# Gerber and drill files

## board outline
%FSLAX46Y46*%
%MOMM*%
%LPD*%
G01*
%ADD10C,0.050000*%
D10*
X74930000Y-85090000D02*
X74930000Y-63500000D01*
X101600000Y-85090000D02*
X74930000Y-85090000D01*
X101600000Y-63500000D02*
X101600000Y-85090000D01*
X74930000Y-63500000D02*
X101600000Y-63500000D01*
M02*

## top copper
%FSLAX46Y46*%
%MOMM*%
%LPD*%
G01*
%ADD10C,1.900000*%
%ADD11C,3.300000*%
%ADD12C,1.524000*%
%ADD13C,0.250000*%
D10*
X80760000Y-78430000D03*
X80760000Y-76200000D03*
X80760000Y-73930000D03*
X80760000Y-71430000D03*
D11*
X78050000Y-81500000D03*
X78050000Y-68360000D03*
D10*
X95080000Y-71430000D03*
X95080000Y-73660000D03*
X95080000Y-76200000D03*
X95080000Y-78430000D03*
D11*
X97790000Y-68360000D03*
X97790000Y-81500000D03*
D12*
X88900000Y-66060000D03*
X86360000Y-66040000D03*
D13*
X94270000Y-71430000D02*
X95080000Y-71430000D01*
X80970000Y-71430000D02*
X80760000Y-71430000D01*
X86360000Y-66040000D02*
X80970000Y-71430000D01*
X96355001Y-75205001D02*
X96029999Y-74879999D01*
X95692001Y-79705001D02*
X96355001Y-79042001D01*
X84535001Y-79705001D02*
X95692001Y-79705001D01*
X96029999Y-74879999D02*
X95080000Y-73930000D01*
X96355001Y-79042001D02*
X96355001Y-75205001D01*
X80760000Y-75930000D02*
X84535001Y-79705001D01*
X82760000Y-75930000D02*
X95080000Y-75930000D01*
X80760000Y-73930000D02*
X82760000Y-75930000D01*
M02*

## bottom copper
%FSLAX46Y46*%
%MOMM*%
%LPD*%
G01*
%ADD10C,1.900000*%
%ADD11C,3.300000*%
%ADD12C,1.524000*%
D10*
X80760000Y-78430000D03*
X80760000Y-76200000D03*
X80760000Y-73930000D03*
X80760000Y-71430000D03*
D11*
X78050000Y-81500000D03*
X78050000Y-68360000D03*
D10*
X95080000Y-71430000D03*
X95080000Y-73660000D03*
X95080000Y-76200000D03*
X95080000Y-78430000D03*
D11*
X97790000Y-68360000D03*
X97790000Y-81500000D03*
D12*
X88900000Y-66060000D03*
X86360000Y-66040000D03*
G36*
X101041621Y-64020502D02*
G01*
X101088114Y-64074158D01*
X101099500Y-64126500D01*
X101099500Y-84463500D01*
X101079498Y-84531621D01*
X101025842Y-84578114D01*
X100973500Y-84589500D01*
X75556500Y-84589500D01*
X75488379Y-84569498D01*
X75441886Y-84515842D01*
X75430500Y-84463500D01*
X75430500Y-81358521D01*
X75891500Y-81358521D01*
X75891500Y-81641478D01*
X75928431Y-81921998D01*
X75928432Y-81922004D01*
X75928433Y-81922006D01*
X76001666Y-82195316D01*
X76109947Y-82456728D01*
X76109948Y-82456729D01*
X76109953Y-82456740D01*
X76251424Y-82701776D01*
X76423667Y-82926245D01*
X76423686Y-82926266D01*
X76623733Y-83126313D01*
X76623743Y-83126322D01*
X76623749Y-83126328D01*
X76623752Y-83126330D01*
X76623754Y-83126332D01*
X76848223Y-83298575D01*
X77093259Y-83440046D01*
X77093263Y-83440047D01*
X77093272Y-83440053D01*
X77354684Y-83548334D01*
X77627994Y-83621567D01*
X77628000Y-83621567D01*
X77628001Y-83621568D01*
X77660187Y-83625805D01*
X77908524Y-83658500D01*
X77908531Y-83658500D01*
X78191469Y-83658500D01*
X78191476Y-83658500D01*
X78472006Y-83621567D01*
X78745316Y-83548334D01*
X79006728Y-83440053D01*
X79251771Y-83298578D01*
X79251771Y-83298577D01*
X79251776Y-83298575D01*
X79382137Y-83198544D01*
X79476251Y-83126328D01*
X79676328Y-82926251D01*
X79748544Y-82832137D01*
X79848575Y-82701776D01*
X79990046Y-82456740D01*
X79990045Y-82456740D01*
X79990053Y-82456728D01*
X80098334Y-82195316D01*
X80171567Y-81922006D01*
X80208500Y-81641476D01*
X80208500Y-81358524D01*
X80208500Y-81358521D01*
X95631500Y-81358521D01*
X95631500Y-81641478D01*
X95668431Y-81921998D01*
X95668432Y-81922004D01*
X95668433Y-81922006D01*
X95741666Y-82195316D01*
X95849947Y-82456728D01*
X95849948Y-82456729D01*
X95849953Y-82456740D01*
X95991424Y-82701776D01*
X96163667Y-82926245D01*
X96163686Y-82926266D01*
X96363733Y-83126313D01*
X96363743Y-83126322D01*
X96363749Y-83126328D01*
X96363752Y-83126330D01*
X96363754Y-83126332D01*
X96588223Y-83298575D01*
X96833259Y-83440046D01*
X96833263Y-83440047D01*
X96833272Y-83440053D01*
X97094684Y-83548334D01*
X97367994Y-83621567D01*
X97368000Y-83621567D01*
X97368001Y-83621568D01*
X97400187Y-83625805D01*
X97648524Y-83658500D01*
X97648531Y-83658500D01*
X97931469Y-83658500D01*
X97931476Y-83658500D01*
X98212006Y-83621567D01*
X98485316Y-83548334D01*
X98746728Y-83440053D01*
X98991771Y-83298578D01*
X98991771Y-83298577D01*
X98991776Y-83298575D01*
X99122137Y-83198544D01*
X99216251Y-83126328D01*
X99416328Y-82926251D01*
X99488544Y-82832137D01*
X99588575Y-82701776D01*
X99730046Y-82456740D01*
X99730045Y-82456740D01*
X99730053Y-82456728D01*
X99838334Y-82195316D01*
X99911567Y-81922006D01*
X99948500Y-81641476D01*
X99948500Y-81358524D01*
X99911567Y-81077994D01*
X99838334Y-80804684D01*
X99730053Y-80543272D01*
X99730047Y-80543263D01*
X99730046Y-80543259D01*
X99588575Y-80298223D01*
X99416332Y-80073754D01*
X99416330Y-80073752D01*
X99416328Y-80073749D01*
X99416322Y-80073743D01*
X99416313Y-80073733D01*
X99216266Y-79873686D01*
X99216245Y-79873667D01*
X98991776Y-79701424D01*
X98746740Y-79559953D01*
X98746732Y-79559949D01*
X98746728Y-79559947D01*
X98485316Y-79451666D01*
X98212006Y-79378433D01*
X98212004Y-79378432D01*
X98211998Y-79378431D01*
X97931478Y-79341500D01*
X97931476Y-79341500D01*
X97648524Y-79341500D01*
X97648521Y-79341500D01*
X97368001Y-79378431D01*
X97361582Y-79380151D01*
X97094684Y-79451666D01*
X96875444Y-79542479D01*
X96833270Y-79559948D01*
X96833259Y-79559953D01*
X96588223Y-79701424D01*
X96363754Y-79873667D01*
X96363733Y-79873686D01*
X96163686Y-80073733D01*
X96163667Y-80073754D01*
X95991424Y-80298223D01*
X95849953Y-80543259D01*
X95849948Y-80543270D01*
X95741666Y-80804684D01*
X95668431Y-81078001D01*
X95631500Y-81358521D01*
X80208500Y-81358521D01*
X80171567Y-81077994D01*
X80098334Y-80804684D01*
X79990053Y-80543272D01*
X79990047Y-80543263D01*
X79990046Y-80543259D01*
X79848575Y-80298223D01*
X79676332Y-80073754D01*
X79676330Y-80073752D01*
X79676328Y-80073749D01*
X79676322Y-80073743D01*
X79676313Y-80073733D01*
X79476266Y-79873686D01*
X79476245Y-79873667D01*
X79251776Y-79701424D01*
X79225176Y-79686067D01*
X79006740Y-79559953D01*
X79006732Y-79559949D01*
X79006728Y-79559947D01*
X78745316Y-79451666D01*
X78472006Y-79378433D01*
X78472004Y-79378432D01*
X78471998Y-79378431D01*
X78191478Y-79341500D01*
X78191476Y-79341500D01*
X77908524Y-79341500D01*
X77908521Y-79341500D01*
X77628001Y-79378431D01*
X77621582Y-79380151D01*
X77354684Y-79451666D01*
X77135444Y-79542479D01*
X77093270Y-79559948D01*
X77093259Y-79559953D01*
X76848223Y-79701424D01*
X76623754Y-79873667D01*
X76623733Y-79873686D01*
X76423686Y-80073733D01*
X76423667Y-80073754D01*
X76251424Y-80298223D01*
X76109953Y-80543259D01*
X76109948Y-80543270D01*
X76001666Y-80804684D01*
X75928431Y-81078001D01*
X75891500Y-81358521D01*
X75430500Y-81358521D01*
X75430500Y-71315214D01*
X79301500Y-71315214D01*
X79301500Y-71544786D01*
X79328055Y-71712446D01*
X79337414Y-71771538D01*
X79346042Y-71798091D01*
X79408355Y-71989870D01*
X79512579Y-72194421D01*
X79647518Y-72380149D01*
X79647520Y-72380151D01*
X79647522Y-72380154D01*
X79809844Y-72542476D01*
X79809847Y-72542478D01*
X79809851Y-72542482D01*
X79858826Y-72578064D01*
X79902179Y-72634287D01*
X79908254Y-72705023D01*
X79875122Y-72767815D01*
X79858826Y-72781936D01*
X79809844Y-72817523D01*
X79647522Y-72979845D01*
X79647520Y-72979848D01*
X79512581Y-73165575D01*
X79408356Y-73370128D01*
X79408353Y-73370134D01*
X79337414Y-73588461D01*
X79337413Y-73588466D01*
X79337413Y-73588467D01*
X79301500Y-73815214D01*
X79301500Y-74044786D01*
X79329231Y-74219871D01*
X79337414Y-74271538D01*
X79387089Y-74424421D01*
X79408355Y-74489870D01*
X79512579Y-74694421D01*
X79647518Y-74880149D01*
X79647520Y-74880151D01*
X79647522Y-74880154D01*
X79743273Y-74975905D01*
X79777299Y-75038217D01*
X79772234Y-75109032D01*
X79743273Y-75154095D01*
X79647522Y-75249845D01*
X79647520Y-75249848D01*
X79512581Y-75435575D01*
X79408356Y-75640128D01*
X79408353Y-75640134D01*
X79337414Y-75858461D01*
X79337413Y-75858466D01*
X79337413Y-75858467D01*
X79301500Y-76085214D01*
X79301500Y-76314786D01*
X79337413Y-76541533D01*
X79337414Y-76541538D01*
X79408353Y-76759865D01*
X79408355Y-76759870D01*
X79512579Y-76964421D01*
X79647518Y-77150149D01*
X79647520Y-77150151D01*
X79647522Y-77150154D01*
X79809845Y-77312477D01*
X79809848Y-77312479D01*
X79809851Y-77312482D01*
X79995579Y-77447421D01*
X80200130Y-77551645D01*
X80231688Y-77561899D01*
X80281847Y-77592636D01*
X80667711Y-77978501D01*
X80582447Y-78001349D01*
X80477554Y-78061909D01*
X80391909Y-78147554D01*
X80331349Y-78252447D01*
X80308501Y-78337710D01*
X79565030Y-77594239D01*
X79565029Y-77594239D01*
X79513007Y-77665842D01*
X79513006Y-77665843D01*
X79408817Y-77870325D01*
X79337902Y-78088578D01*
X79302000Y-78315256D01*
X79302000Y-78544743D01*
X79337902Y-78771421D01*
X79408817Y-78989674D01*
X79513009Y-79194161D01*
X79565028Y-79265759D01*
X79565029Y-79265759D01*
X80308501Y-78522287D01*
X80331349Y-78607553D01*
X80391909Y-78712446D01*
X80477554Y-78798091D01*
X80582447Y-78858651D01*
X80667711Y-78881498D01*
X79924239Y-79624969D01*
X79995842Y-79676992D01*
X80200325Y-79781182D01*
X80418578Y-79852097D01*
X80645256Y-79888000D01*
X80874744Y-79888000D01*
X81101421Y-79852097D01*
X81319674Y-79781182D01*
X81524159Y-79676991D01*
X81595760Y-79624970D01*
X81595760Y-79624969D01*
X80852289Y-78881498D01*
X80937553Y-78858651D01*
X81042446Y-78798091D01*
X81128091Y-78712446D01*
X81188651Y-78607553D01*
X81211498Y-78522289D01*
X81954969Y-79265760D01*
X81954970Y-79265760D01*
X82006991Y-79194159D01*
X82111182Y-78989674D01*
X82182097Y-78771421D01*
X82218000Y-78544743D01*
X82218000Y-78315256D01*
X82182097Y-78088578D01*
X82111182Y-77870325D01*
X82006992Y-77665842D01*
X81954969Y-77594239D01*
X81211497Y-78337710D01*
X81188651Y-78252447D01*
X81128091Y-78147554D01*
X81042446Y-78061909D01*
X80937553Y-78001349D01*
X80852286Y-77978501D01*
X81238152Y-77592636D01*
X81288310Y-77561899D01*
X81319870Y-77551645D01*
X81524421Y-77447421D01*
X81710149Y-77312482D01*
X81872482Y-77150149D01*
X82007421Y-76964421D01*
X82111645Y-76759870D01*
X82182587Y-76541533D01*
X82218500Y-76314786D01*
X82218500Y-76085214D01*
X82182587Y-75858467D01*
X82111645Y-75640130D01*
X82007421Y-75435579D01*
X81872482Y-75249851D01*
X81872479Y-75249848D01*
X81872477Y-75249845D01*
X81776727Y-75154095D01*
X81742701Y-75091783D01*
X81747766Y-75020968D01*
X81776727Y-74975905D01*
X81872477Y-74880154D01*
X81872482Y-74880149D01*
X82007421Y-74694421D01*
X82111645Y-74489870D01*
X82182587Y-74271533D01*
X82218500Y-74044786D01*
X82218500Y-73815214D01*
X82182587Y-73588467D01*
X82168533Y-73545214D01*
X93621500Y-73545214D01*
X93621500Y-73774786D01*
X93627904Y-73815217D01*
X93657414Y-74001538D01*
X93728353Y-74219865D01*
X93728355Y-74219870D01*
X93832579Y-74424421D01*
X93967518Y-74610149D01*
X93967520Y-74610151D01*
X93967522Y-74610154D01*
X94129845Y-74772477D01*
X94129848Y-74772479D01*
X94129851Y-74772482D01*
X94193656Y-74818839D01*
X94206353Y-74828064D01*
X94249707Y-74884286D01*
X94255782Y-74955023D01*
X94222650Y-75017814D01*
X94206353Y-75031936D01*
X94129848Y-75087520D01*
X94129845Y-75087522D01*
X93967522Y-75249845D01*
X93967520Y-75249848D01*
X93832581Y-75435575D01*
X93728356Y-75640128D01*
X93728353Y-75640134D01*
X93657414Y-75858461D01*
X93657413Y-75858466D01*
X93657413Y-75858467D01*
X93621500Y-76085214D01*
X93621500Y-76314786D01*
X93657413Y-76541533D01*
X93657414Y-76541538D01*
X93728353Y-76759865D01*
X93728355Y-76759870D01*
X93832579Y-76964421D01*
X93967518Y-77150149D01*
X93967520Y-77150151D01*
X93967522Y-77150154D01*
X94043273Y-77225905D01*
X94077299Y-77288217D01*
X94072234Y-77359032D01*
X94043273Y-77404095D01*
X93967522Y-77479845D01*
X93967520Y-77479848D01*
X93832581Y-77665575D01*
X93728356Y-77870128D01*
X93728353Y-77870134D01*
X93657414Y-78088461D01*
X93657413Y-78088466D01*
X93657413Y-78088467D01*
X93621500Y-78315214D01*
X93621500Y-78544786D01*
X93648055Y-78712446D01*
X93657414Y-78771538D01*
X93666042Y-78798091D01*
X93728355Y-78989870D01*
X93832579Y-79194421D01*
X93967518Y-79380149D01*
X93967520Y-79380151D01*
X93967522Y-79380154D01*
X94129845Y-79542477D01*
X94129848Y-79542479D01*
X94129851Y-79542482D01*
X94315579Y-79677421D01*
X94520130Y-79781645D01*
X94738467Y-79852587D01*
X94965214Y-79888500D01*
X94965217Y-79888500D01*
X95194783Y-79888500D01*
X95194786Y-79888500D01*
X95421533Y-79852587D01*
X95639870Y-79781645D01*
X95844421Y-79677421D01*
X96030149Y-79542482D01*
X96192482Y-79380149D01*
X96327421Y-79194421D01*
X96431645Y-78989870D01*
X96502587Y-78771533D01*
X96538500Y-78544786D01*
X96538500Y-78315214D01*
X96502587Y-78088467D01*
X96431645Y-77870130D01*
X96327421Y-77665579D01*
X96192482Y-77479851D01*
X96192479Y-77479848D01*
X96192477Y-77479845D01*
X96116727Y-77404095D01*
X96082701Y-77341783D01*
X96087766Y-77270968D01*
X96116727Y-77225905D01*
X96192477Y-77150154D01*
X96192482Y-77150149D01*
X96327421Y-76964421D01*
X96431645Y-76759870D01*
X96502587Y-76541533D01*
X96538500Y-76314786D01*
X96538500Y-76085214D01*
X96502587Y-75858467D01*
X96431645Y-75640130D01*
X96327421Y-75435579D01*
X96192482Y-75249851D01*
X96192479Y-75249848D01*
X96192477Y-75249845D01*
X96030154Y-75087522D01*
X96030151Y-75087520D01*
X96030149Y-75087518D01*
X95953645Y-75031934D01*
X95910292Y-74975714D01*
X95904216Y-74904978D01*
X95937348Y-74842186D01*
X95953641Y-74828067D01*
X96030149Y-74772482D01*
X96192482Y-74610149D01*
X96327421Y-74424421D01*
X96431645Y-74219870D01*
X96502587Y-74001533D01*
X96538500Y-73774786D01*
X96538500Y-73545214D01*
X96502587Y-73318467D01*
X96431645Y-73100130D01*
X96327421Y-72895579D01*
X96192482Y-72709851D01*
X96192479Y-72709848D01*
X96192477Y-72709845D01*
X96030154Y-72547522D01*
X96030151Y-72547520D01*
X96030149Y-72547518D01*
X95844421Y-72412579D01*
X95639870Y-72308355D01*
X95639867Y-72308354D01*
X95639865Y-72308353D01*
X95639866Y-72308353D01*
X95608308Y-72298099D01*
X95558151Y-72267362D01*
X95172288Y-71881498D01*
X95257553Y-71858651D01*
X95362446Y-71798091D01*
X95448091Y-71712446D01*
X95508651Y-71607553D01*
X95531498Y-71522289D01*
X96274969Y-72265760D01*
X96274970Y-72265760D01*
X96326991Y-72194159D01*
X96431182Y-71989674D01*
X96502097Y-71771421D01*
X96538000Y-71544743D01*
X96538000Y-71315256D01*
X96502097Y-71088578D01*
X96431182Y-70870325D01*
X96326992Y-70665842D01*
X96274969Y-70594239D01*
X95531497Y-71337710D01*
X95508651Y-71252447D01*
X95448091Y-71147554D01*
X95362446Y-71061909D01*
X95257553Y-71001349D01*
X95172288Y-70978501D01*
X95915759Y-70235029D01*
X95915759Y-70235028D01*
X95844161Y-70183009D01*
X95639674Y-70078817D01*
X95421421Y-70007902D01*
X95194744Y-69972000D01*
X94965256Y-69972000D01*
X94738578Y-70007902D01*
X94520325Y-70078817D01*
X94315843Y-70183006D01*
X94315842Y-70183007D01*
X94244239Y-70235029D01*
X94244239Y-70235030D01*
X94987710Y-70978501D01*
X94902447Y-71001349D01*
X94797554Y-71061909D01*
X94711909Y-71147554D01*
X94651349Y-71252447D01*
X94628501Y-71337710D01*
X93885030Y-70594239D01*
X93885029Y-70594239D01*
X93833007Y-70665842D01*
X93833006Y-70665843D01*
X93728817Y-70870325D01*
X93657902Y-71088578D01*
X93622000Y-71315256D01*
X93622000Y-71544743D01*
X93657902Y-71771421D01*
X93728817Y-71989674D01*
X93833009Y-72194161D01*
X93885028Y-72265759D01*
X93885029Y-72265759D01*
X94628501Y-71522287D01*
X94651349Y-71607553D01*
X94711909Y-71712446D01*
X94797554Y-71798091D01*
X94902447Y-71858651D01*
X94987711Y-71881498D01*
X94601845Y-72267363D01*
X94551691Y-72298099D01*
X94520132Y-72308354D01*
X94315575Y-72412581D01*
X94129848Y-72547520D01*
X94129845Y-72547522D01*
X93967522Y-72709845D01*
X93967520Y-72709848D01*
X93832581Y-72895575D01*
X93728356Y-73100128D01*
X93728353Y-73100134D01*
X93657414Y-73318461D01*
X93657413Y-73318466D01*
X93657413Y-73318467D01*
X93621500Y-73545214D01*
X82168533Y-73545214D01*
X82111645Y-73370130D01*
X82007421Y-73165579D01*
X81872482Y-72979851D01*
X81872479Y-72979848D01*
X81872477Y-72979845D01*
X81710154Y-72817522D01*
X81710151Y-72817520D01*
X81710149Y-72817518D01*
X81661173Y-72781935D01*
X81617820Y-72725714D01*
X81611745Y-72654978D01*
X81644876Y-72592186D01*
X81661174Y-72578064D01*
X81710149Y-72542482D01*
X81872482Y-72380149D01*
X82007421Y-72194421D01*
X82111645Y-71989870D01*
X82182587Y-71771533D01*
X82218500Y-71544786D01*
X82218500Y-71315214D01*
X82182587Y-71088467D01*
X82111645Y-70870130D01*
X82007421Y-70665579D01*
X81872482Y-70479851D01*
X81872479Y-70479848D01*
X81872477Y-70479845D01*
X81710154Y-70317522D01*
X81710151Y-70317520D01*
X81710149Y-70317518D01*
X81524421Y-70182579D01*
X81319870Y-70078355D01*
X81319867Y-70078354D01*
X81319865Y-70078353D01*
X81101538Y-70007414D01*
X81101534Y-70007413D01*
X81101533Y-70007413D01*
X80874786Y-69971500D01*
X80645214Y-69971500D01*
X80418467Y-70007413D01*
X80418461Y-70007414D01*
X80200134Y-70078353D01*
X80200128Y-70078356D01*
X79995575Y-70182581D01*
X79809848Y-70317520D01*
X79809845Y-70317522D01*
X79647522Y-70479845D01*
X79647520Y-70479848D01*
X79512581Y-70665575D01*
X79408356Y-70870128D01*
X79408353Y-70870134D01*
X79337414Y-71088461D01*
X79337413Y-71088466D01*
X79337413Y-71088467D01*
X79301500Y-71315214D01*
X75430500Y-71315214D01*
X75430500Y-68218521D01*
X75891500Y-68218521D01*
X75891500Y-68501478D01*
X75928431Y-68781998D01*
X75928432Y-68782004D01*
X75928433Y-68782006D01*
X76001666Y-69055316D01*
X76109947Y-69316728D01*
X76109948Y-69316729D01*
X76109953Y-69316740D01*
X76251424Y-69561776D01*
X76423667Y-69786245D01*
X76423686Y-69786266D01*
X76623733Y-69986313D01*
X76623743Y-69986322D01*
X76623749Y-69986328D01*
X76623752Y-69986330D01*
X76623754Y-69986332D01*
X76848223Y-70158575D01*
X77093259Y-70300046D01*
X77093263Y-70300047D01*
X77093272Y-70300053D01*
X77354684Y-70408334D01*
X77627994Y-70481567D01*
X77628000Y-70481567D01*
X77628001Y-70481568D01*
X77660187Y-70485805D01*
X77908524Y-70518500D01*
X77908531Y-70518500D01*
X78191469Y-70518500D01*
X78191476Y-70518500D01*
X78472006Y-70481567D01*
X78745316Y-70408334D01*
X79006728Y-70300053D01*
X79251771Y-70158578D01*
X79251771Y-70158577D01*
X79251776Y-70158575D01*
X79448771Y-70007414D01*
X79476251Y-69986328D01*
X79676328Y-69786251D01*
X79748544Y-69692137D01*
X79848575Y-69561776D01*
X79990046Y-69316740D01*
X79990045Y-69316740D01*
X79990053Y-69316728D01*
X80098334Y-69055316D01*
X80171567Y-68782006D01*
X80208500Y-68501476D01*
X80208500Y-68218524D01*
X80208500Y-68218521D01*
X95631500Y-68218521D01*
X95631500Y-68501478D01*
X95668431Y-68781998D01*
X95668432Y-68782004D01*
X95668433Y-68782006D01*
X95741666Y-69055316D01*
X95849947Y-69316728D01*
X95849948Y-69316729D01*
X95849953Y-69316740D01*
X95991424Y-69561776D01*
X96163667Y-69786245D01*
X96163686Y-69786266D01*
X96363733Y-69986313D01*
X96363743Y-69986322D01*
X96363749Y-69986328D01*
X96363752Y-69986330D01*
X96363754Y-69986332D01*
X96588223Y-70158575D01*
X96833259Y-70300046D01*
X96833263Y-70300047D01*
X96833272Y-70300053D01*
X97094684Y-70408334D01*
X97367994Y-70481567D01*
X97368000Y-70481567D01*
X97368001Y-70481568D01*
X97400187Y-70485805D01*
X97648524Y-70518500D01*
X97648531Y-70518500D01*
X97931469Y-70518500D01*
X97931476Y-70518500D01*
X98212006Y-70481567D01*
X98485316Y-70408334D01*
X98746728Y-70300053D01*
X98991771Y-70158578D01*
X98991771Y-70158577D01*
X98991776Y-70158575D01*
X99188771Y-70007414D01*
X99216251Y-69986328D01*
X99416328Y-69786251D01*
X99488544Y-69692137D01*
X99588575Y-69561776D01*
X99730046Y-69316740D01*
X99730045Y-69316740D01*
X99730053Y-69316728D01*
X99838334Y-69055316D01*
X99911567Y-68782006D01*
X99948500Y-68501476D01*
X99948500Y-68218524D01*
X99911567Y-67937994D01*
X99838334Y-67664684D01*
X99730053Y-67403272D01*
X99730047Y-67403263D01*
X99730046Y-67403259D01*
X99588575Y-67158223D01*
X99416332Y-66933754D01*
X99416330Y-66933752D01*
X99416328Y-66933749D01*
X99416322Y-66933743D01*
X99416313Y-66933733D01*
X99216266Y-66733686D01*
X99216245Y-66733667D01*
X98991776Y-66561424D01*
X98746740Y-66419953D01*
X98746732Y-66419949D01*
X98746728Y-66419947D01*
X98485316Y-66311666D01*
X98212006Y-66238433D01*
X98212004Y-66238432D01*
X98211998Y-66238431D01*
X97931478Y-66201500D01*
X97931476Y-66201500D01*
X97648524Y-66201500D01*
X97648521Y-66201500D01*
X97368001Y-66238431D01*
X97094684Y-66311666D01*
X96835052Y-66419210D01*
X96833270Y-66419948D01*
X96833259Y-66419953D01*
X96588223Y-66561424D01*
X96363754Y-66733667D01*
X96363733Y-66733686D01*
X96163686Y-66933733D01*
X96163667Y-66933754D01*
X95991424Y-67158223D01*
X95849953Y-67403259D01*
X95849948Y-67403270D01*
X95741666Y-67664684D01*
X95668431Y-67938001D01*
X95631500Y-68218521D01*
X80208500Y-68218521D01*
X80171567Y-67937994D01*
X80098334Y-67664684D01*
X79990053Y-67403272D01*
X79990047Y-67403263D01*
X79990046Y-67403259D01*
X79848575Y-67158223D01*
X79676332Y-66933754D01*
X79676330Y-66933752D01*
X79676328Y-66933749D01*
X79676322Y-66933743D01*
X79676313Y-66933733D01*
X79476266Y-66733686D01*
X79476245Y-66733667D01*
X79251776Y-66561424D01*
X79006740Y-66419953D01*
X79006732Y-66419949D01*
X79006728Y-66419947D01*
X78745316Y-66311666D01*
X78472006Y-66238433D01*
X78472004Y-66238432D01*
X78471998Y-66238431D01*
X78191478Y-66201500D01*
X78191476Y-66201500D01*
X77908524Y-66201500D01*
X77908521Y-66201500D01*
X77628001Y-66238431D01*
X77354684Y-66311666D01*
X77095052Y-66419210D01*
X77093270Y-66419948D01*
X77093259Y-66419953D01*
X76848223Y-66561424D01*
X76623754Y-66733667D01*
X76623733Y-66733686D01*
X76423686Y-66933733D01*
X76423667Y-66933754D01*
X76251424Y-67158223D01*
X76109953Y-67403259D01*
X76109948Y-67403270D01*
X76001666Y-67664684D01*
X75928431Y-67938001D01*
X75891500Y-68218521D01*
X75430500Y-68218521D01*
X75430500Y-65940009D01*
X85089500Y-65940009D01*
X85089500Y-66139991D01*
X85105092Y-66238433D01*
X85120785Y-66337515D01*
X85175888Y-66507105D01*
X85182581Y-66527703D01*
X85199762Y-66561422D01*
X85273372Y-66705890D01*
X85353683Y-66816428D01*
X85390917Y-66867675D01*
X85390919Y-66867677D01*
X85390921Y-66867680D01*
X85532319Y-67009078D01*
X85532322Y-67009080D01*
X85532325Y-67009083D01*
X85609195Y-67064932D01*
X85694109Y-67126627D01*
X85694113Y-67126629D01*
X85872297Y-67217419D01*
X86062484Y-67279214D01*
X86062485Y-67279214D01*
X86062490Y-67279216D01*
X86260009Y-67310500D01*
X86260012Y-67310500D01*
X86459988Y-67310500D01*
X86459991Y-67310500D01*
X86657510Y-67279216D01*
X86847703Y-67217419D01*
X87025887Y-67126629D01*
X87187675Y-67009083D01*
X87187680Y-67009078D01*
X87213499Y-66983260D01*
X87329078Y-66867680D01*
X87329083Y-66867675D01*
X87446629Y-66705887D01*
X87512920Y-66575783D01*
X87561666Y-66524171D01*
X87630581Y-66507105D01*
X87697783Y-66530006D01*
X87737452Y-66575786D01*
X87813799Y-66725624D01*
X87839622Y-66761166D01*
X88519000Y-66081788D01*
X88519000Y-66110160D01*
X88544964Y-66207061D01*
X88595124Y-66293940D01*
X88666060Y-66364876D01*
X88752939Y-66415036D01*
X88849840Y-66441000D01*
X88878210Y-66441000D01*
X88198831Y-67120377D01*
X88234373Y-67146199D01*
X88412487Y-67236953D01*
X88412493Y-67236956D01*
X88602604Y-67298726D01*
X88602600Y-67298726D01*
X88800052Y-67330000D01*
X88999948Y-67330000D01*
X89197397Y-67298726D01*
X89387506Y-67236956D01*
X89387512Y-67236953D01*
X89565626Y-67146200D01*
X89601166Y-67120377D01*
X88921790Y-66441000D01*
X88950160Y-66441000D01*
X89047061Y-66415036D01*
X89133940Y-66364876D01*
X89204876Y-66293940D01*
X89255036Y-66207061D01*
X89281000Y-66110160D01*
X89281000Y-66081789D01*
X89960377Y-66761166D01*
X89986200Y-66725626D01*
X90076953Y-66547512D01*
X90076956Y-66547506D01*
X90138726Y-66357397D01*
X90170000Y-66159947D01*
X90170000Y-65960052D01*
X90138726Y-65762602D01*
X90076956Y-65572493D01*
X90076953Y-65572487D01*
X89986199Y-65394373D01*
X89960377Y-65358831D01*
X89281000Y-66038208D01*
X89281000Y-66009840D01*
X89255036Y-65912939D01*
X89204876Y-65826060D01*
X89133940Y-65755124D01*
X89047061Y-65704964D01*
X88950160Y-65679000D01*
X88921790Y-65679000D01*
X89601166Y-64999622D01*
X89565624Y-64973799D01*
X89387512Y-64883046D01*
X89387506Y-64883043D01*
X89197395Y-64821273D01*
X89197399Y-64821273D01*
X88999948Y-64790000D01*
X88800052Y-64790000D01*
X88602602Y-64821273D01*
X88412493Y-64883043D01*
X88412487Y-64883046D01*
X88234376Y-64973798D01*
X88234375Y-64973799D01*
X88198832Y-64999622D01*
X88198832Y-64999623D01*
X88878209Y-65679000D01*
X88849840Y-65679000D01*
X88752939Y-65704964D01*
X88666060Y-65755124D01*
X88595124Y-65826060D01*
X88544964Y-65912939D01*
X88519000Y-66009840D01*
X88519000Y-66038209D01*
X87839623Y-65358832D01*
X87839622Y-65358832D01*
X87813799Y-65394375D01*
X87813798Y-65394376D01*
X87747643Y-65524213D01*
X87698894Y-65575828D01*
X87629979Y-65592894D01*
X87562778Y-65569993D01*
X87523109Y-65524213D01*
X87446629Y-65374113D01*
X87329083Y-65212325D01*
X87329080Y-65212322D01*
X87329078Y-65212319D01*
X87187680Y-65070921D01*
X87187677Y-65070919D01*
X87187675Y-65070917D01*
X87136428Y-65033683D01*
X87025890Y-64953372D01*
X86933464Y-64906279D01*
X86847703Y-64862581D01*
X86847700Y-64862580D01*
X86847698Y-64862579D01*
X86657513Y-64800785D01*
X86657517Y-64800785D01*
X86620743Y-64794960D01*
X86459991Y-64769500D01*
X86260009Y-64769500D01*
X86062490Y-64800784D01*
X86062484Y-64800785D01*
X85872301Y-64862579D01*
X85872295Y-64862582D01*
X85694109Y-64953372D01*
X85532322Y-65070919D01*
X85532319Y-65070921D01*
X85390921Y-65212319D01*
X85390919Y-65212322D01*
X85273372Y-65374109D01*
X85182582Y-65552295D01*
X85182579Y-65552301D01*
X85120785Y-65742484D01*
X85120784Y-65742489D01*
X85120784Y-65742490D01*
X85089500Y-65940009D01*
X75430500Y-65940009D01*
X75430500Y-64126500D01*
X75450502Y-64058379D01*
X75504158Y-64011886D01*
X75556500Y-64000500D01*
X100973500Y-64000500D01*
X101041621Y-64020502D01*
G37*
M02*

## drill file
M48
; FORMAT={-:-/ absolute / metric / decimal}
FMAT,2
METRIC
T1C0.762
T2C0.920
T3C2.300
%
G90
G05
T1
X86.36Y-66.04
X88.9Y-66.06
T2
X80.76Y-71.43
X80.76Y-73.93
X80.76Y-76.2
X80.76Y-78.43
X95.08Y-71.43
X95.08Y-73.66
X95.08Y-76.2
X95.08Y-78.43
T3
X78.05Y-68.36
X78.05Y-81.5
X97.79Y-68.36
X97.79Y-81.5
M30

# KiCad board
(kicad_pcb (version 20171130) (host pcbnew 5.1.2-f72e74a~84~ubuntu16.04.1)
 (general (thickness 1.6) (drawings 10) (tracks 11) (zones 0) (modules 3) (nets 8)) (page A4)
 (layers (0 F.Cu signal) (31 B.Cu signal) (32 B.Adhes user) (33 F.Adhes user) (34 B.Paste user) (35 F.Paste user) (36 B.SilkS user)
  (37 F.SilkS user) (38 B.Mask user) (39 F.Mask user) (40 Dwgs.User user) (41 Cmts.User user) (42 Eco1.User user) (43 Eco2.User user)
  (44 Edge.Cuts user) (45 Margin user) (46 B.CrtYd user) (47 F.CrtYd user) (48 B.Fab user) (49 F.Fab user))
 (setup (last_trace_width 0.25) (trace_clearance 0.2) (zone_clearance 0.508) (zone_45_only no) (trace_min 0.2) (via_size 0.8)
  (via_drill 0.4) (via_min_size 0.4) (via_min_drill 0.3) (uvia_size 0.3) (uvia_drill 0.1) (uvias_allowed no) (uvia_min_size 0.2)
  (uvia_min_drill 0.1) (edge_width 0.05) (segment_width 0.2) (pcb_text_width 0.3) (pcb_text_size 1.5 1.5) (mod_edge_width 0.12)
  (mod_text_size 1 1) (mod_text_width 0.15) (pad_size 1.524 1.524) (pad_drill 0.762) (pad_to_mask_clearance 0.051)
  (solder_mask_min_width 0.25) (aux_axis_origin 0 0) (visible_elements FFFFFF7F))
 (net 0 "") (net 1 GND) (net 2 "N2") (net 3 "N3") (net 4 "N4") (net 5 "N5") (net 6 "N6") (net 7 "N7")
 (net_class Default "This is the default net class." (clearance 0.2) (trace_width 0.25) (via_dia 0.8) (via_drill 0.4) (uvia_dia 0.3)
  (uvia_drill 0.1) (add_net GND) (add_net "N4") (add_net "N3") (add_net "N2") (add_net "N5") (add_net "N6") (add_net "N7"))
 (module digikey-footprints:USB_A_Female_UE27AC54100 (layer F.Cu) (at 78.05 74.93 270)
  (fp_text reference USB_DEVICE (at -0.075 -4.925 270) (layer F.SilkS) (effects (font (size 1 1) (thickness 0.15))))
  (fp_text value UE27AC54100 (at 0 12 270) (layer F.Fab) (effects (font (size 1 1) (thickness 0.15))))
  (pad 4 thru_hole circle (at 3.5 -2.71 270) (size 1.9 1.9) (drill 0.92) (layers *.Cu *.Mask) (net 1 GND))
  (pad 3 thru_hole circle (at 1.27 -2.71 270) (size 1.9 1.9) (drill 0.92) (layers *.Cu *.Mask) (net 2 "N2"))
  (pad 2 thru_hole circle (at -1 -2.71 270) (size 1.9 1.9) (drill 0.92) (layers *.Cu *.Mask) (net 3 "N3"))
  (pad 1 thru_hole circle (at -3.5 -2.71 270) (size 1.9 1.9) (drill 0.92) (layers *.Cu *.Mask) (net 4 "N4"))
  (pad SH thru_hole circle (at 6.57 0 270) (size 3.3 3.3) (drill 2.3) (layers *.Cu *.Mask) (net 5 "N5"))
  (pad SH thru_hole circle (at -6.57 0 270) (size 3.3 3.3) (drill 2.3) (layers *.Cu *.Mask) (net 5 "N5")))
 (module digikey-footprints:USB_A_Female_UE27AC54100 (layer F.Cu) (at 97.79 74.93 90)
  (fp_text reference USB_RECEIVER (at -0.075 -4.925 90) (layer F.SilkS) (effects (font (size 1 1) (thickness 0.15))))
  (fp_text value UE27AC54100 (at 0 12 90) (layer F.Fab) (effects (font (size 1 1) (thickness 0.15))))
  (pad 4 thru_hole circle (at 3.5 -2.71 90) (size 1.9 1.9) (drill 0.92) (layers *.Cu *.Mask) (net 1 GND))
  (pad 3 thru_hole circle (at 1.27 -2.71 90) (size 1.9 1.9) (drill 0.92) (layers *.Cu *.Mask) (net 2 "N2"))
  (pad 2 thru_hole circle (at -1.27 -2.71 90) (size 1.9 1.9) (drill 0.92) (layers *.Cu *.Mask) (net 3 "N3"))
  (pad 1 thru_hole circle (at -3.5 -2.71 90) (size 1.9 1.9) (drill 0.92) (layers *.Cu *.Mask) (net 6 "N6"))
  (pad SH thru_hole circle (at 6.57 0 90) (size 3.3 3.3) (drill 2.3) (layers *.Cu *.Mask) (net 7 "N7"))
  (pad SH thru_hole circle (at -6.57 0 90) (size 3.3 3.3) (drill 2.3) (layers *.Cu *.Mask) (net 7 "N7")))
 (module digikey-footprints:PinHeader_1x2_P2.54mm (layer F.Cu) (at 86.36 66.04)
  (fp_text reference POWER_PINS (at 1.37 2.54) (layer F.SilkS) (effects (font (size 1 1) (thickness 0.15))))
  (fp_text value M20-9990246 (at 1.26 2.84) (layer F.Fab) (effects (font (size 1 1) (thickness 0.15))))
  (pad 2 thru_hole circle (at 2.54 0.02) (size 1.524 1.524) (drill 0.762) (layers *.Cu *.Mask) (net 1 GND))
  (pad 1 thru_hole circle (at 0 0) (size 1.524 1.524) (drill 0.762) (layers *.Cu *.Mask) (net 4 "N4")))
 (gr_line (start 74.93 85.09) (end 74.93 63.5) (layer Edge.Cuts) (width 0.05))
 (gr_line (start 101.6 85.09) (end 74.93 85.09) (layer Edge.Cuts) (width 0.05))
 (gr_line (start 101.6 63.5) (end 101.6 85.09) (layer Edge.Cuts) (width 0.05))
 (gr_line (start 74.93 63.5) (end 101.6 63.5) (layer Edge.Cuts) (width 0.05))
 (segment (start 94.27 71.43) (end 95.08 71.43) (width 0.25) (layer F.Cu) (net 1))
 (segment (start 80.97 71.43) (end 80.76 71.43) (width 0.25) (layer F.Cu) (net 4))
 (segment (start 86.36 66.04) (end 80.97 71.43) (width 0.25) (layer F.Cu) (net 4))
 (segment (start 96.355001 75.205001) (end 96.029999 74.879999) (width 0.25) (layer F.Cu) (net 2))
 (segment (start 95.692001 79.705001) (end 96.355001 79.042001) (width 0.25) (layer F.Cu) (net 2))
 (segment (start 84.535001 79.705001) (end 95.692001 79.705001) (width 0.25) (layer F.Cu) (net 2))
 (segment (start 96.029999 74.879999) (end 95.08 73.93) (width 0.25) (layer F.Cu) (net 2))
 (segment (start 96.355001 79.042001) (end 96.355001 75.205001) (width 0.25) (layer F.Cu) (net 2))
 (segment (start 80.76 75.93) (end 84.535001 79.705001) (width 0.25) (layer F.Cu) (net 2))
 (segment (start 82.76 75.93) (end 95.08 75.93) (width 0.25) (layer F.Cu) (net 3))
 (segment (start 80.76 73.93) (end 82.76 75.93) (width 0.25) (layer F.Cu) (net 3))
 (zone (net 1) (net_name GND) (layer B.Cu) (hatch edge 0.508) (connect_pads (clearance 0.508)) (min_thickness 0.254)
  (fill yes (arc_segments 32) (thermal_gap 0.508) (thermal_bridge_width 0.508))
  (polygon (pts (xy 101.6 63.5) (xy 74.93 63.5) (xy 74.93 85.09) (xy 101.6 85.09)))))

